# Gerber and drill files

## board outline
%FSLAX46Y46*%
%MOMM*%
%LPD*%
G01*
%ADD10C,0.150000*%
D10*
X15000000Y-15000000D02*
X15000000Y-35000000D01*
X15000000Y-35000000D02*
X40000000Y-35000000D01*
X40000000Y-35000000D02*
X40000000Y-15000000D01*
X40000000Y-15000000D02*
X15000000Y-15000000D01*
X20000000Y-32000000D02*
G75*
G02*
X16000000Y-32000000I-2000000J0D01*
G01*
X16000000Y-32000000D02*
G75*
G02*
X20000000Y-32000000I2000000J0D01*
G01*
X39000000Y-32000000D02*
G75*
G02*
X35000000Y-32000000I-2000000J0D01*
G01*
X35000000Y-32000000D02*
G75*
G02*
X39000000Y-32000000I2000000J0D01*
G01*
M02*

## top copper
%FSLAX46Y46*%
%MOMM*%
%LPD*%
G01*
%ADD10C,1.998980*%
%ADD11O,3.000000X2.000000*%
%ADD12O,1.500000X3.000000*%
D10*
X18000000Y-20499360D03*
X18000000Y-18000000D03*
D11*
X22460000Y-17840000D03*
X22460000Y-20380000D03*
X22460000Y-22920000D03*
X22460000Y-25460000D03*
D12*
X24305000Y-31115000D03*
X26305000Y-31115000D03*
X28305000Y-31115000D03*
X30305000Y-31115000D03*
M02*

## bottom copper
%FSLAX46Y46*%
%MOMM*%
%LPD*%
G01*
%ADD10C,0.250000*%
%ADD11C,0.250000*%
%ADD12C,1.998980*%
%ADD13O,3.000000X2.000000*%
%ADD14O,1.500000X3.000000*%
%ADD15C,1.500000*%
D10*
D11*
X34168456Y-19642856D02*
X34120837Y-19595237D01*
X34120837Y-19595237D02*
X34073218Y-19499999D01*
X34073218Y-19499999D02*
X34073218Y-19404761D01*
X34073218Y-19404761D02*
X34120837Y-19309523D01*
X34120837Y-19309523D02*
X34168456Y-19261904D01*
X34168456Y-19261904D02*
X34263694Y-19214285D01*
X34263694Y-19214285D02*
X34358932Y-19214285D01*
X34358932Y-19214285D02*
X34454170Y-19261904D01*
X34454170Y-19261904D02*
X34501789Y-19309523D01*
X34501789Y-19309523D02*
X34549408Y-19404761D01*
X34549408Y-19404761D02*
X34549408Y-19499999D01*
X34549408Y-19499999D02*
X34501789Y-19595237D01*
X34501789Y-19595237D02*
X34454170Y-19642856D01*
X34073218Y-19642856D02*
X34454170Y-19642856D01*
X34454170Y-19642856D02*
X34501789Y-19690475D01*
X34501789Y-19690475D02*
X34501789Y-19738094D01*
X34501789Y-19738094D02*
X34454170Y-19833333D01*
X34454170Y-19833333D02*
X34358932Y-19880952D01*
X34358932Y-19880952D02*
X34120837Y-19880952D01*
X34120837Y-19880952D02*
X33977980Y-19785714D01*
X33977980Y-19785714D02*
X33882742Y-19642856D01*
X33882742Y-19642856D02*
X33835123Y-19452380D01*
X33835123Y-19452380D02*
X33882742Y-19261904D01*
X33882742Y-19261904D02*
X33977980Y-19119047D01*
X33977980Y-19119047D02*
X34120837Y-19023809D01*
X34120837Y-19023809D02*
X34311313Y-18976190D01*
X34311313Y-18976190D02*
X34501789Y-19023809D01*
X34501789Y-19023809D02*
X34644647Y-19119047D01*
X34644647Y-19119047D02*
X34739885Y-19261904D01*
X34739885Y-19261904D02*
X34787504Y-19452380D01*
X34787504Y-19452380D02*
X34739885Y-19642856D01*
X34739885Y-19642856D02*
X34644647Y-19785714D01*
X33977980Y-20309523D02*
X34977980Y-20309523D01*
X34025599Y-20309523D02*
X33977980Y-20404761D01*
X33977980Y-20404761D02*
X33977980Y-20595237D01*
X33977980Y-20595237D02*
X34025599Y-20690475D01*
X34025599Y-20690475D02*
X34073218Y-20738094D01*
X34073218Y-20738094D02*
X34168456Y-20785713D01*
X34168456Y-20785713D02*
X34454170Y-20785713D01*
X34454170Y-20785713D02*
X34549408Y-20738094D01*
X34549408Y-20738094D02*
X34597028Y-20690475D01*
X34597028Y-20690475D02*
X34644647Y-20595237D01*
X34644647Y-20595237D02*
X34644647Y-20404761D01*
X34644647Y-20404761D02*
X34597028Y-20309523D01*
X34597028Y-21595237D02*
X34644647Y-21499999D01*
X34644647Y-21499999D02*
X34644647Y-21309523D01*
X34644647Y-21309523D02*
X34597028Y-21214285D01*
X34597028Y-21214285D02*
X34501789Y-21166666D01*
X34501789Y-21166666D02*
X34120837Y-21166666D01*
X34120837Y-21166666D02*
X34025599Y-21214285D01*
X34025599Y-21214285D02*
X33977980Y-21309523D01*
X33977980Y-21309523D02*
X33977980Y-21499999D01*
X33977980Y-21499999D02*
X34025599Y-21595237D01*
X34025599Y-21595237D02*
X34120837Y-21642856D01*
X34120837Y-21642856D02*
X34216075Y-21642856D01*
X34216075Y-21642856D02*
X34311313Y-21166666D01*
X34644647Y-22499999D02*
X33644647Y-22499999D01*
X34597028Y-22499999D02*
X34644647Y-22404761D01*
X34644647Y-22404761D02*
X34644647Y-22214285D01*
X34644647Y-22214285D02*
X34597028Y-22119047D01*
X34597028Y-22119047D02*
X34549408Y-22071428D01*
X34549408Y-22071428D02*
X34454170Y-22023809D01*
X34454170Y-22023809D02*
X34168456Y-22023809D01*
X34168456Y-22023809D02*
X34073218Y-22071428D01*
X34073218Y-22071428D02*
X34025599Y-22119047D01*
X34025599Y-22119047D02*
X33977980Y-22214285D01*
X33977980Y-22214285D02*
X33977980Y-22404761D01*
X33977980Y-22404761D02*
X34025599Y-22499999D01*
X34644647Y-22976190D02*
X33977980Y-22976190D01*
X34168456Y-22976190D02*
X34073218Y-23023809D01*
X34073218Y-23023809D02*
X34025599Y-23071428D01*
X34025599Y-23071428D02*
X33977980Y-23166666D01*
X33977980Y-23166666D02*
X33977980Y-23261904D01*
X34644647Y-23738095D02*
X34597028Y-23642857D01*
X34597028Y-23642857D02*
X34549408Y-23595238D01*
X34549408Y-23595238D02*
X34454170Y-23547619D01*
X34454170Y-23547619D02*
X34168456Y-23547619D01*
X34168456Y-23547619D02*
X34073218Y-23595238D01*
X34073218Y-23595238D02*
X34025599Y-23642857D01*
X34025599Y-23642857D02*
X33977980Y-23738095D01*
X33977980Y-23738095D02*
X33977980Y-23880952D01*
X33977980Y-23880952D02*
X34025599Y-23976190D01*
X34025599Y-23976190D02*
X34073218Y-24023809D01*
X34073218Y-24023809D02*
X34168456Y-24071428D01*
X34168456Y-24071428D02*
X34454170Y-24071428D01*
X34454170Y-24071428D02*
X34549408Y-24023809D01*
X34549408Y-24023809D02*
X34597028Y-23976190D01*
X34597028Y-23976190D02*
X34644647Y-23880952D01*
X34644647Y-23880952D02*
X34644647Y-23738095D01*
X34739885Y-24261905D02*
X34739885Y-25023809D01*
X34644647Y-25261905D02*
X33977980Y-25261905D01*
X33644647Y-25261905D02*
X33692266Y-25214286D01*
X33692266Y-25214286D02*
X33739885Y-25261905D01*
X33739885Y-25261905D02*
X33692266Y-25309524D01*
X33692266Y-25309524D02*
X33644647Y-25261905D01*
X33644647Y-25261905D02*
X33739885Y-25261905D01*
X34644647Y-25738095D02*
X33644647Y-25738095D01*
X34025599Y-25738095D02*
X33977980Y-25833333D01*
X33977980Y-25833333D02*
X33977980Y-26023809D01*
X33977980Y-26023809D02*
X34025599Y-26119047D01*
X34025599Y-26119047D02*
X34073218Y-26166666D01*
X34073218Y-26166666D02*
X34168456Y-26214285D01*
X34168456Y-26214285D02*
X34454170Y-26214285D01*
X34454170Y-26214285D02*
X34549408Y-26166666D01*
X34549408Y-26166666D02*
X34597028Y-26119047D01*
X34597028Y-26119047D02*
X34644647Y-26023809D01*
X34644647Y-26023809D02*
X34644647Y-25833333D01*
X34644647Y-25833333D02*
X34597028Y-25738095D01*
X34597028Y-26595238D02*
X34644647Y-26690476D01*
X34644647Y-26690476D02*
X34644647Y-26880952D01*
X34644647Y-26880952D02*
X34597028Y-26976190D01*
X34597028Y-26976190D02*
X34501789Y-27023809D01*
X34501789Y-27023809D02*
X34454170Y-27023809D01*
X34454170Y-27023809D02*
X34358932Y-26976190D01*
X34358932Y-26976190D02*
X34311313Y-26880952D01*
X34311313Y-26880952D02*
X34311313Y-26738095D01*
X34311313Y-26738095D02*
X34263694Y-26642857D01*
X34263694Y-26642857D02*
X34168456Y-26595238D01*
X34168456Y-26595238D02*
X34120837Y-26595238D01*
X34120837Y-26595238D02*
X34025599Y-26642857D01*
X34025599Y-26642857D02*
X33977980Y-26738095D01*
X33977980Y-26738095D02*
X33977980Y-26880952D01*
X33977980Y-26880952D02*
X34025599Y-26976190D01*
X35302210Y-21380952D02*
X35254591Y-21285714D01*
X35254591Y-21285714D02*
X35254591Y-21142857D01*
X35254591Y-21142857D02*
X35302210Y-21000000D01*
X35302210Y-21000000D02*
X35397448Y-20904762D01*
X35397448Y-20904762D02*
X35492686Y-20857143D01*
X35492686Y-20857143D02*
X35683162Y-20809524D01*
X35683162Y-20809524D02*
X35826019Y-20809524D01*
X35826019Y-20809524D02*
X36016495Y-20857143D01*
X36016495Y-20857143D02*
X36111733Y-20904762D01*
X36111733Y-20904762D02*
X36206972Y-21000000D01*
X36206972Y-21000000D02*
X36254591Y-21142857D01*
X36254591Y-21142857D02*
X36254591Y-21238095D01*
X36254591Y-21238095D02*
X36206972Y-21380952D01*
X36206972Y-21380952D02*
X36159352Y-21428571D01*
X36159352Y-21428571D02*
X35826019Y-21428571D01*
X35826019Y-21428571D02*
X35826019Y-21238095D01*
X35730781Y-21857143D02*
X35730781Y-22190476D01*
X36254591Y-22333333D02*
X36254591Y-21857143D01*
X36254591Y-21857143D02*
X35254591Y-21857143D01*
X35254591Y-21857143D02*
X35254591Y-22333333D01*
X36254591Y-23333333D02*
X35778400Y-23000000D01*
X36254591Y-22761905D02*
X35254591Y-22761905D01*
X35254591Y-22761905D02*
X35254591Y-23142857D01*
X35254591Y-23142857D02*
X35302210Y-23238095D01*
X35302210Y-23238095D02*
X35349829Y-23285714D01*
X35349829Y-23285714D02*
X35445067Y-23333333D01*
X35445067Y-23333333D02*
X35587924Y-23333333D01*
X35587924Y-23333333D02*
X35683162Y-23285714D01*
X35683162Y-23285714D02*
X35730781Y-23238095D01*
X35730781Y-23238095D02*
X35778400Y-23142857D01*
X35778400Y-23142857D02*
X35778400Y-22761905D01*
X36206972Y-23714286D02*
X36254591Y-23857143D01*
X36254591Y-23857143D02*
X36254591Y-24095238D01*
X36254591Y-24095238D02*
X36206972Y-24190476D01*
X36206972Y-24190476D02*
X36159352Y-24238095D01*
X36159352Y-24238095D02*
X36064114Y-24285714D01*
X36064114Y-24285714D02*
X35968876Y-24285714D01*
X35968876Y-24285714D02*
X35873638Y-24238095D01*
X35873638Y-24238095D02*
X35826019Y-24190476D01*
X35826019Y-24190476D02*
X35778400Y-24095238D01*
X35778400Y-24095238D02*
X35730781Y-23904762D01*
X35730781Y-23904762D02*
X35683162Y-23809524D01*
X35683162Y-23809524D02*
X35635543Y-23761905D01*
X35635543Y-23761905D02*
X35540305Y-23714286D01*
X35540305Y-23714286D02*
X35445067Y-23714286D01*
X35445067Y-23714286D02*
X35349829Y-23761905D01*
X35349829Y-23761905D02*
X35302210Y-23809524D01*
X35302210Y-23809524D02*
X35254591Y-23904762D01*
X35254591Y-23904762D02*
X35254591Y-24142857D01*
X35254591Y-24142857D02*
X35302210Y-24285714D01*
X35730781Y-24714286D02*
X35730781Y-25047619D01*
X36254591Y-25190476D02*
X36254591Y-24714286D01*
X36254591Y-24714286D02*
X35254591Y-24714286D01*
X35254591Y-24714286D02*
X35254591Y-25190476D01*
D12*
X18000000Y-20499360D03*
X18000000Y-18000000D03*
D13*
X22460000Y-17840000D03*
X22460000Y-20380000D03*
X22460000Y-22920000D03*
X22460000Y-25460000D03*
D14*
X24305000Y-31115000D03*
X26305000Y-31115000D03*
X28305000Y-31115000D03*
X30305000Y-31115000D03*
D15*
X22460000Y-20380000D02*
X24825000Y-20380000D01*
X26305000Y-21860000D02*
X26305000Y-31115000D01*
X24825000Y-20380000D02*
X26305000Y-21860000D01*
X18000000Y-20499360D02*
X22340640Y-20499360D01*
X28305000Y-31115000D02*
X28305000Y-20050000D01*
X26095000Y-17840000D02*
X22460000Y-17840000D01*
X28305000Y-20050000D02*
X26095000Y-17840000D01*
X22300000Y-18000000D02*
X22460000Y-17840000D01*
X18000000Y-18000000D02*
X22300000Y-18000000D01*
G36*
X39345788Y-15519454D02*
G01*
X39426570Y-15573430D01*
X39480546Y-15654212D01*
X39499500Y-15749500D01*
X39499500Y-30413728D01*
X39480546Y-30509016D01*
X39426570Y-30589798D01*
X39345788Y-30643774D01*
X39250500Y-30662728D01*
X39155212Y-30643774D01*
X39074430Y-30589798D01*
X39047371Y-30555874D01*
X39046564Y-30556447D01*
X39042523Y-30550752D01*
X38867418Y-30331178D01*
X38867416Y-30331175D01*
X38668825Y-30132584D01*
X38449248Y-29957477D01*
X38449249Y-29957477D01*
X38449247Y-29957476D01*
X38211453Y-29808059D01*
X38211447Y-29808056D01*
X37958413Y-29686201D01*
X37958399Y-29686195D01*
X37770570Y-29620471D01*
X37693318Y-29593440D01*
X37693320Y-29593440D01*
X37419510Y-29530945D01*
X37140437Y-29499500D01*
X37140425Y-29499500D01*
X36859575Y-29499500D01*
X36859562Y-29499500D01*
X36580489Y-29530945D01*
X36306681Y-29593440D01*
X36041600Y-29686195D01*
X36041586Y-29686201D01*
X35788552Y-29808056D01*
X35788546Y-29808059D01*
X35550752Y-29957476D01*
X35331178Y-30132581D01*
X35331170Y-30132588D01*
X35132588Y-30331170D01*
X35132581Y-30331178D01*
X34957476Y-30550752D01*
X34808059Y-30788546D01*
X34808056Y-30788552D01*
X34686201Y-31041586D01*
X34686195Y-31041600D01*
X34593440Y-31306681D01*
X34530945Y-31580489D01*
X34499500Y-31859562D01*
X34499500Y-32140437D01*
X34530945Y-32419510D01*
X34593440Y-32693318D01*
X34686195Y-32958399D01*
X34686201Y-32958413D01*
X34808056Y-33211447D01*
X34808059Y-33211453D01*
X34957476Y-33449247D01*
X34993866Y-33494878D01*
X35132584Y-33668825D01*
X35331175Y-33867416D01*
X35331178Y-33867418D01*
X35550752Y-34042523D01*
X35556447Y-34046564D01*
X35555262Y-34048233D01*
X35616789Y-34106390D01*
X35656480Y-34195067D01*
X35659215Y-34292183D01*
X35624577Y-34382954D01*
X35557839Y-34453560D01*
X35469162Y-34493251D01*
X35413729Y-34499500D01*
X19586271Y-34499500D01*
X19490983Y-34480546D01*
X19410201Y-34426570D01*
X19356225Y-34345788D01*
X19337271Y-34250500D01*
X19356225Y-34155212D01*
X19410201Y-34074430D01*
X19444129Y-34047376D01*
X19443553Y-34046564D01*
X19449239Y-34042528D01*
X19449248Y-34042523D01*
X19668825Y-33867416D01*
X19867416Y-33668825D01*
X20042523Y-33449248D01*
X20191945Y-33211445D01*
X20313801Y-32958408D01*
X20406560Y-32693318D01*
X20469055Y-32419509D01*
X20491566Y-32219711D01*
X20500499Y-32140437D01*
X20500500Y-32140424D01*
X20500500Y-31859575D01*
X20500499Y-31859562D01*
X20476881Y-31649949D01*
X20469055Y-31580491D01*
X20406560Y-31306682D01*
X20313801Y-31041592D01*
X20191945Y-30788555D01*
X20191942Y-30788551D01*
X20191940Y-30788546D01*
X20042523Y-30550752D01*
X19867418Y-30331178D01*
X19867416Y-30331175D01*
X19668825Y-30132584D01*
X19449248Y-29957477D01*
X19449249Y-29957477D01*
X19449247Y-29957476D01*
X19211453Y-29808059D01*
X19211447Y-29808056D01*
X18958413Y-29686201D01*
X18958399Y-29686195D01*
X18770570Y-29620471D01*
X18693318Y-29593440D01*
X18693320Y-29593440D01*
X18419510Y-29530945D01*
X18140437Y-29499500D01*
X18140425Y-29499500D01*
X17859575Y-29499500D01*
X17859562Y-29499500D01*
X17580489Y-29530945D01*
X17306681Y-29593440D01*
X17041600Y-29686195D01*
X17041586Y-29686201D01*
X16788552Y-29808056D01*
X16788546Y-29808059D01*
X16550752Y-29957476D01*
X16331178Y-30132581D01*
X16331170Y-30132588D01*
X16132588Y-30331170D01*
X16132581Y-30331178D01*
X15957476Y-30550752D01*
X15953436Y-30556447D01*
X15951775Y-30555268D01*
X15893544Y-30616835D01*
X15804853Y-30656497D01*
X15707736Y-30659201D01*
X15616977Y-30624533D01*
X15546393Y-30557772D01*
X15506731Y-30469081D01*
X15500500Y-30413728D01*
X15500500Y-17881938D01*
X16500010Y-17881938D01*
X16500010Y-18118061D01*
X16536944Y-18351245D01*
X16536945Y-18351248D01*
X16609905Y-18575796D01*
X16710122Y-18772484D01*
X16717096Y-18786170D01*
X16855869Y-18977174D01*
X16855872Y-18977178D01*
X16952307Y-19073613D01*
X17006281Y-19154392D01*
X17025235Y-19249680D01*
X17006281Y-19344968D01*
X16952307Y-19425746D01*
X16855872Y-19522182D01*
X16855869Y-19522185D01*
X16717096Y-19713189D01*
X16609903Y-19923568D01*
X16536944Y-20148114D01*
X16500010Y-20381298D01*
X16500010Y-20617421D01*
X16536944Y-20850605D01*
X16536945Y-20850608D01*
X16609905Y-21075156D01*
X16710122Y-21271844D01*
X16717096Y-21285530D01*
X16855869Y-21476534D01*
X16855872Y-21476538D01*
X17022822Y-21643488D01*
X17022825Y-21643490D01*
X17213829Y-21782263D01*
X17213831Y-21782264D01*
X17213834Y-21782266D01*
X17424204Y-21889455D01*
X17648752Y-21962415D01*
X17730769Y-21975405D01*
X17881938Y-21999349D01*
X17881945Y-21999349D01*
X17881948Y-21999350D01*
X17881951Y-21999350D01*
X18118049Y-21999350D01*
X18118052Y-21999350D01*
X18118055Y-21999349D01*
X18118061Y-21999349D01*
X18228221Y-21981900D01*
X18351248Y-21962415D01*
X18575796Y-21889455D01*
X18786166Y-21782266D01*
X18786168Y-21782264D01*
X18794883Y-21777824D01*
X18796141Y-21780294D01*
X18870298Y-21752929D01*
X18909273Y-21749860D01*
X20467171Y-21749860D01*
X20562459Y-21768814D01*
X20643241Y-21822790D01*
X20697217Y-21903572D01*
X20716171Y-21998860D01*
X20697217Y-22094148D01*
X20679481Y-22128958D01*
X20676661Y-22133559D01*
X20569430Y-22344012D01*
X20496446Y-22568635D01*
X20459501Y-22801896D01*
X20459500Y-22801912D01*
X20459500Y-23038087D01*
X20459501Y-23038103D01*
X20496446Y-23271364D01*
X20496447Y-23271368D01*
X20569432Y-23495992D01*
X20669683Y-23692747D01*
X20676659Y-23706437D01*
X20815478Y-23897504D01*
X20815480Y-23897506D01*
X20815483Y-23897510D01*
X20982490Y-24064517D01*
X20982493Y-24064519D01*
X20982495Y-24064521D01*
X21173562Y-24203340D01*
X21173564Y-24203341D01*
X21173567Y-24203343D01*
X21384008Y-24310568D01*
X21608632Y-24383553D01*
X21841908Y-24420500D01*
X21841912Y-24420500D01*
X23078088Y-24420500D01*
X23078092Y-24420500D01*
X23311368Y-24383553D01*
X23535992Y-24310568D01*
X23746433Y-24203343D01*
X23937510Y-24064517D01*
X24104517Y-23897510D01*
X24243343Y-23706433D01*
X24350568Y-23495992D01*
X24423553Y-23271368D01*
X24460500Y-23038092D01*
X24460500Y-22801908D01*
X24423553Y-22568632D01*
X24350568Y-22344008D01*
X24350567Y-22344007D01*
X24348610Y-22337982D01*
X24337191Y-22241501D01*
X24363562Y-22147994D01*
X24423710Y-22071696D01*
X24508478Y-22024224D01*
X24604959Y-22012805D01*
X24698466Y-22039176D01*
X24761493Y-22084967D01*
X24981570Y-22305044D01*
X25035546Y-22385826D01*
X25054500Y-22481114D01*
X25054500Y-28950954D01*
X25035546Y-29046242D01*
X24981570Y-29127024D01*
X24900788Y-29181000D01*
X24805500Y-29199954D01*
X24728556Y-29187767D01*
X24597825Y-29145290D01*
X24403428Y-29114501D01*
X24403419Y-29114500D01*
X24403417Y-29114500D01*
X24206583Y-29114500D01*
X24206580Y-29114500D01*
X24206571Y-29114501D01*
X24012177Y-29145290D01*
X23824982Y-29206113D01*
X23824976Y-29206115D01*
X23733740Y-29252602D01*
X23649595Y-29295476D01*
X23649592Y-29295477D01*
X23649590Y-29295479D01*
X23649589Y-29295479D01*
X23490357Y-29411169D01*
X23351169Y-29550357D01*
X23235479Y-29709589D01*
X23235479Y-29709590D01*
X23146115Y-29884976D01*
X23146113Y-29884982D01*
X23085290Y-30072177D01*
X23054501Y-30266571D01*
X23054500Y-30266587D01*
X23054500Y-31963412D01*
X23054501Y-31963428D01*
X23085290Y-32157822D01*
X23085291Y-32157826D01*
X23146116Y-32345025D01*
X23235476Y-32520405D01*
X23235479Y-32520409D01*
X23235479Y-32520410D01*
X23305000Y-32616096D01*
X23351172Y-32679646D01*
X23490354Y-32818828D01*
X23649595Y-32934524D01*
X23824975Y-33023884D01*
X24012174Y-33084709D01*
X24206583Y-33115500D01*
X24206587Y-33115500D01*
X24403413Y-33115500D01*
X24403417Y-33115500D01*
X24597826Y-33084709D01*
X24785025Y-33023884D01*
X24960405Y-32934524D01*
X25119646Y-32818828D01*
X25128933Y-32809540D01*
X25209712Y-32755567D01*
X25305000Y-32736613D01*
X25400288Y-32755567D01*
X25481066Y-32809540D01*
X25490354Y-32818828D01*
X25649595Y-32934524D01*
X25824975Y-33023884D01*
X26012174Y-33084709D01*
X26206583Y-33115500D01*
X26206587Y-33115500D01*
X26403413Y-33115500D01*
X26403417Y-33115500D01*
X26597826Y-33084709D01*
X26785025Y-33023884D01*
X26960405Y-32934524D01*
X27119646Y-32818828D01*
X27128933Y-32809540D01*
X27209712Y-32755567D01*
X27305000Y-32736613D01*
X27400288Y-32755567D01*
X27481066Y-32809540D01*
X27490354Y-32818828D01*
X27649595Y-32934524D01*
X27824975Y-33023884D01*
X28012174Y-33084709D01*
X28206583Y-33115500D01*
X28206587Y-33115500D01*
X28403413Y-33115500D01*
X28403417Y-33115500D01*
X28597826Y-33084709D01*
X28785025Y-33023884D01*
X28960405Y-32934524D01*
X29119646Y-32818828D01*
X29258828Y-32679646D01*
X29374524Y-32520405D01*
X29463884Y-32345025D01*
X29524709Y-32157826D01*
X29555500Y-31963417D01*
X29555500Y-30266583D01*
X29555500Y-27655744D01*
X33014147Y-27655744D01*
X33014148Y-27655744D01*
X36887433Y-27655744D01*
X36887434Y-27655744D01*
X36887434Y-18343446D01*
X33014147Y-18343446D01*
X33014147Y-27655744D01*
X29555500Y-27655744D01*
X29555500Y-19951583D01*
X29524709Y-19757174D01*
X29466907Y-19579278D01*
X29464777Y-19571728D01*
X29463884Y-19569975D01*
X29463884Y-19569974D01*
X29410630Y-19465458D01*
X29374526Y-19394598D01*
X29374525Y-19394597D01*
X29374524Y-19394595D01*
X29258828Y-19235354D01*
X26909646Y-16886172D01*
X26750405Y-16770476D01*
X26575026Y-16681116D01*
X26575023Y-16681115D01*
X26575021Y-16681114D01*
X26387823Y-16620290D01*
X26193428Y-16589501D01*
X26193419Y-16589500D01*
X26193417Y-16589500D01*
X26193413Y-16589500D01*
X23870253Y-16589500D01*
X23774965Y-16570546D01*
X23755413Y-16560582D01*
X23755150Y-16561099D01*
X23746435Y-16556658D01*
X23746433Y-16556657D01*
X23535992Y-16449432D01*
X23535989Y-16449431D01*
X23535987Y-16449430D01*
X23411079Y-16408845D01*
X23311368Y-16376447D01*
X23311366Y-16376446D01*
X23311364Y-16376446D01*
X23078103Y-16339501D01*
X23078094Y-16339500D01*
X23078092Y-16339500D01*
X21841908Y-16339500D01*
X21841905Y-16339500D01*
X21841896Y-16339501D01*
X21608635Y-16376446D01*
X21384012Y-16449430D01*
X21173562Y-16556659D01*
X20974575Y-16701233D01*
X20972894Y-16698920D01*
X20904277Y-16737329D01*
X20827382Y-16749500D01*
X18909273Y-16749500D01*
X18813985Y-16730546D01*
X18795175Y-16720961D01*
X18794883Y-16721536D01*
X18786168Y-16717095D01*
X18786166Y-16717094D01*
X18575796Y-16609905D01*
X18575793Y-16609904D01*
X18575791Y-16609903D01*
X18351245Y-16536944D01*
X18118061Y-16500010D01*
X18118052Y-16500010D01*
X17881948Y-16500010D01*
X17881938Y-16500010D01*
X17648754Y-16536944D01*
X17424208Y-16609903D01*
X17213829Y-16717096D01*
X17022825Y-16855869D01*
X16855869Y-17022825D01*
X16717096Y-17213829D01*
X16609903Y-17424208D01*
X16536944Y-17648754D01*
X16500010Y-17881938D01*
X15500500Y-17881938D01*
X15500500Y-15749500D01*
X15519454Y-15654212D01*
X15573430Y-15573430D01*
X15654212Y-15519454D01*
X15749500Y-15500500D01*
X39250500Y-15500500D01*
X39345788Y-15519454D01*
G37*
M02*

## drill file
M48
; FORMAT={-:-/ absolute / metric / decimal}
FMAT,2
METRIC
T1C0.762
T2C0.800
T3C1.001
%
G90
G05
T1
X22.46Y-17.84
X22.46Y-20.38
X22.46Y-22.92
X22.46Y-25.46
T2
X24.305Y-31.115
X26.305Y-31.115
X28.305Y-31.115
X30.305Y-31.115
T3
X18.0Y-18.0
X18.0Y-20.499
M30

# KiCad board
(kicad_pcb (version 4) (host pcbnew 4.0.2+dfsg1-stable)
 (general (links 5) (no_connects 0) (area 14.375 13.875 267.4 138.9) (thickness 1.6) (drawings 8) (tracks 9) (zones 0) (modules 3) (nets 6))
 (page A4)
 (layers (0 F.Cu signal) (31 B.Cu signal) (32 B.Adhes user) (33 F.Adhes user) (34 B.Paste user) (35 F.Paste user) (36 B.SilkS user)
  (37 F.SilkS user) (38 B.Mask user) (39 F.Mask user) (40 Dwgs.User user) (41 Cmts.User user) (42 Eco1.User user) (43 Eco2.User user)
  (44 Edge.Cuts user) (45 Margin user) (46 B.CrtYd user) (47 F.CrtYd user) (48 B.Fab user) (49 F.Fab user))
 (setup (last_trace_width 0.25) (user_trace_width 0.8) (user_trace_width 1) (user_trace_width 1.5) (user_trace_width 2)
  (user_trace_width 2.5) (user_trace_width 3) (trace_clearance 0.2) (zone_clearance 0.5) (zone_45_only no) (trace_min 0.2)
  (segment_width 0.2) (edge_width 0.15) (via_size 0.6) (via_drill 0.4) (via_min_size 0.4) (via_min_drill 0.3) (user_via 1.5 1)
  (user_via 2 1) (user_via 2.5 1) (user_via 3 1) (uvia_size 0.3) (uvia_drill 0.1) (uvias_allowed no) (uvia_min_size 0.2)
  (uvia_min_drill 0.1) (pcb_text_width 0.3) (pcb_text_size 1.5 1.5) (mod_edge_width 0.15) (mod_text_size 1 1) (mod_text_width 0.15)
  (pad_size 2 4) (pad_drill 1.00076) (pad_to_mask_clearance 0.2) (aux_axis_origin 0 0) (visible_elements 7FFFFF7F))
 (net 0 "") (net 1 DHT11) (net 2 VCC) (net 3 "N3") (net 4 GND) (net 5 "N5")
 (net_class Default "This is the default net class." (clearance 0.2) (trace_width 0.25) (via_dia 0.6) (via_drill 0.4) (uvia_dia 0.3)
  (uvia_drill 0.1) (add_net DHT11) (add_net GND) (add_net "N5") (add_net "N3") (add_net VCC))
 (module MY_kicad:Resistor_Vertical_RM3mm (layer F.Cu) (at 18 18 90)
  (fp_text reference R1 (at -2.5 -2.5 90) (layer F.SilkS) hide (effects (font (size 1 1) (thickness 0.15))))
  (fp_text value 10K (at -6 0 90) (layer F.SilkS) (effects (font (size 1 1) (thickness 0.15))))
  (pad 1 thru_hole circle (at -2.49936 0 90) (size 1.99898 1.99898) (drill 1.00076) (layers *.Cu *.SilkS *.Mask) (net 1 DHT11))
  (pad 2 thru_hole circle (at 0 0 90) (size 1.99898 1.99898) (drill 1.00076) (layers *.Cu *.SilkS *.Mask) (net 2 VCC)))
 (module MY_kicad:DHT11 (layer F.Cu) (at 25 28)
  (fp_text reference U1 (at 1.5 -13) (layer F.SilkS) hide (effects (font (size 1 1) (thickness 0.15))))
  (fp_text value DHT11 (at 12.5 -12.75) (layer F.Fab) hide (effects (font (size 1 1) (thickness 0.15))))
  (pad 1 thru_hole oval (at -2.54 -10.16) (size 3 2) (drill 0.762) (layers *.Cu B.Mask) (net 2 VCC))
  (pad 2 thru_hole oval (at -2.54 -7.62) (size 3 2) (drill 0.762) (layers *.Cu B.Mask) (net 1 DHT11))
  (pad 3 thru_hole oval (at -2.54 -5.08) (size 3 2) (drill 0.762) (layers *.Cu B.Mask) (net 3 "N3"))
  (pad 4 thru_hole oval (at -2.54 -2.54) (size 3 2) (drill 0.762) (layers *.Cu B.Mask) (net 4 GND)))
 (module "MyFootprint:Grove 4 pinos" (layer F.Cu) (at 27.305 31.115)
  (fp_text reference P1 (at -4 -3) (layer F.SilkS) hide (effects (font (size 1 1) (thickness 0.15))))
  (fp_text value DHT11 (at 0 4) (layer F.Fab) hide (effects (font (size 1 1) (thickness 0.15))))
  (pad 1 thru_hole oval (at -3 0) (size 1.5 3) (drill 0.8) (layers *.Cu) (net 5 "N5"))
  (pad 2 thru_hole oval (at -1 0) (size 1.5 3) (drill 0.8) (layers *.Cu) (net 1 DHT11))
  (pad 3 thru_hole oval (at 1 0) (size 1.5 3) (drill 0.8) (layers *.Cu) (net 2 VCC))
  (pad 4 thru_hole oval (at 3 0) (size 1.5 3) (drill 0.8) (layers *.Cu) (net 4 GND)))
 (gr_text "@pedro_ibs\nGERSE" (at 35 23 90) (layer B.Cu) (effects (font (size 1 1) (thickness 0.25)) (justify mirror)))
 (gr_line (start 15 15) (end 15 35) (angle 90) (layer Edge.Cuts) (width 0.15))
 (gr_line (start 15 35) (end 40 35) (angle 90) (layer Edge.Cuts) (width 0.15))
 (gr_line (start 40 35) (end 40 15) (angle 90) (layer Edge.Cuts) (width 0.15))
 (gr_line (start 40 15) (end 15 15) (angle 90) (layer Edge.Cuts) (width 0.15))
 (gr_circle (center 18 32) (end 20 32) (layer Edge.Cuts) (width 0.15))
 (gr_circle (center 37 32) (end 39 32) (layer Edge.Cuts) (width 0.15))
 (segment (start 22.46 20.38) (end 24.825 20.38) (width 1.5) (layer B.Cu) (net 1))
 (segment (start 26.305 21.86) (end 26.305 31.115) (width 1.5) (layer B.Cu) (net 1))
 (segment (start 24.825 20.38) (end 26.305 21.86) (width 1.5) (layer B.Cu) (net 1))
 (segment (start 18 20.49936) (end 22.34064 20.49936) (width 1.5) (layer B.Cu) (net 1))
 (segment (start 28.305 31.115) (end 28.305 20.05) (width 1.5) (layer B.Cu) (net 2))
 (segment (start 26.095 17.84) (end 22.46 17.84) (width 1.5) (layer B.Cu) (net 2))
 (segment (start 28.305 20.05) (end 26.095 17.84) (width 1.5) (layer B.Cu) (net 2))
 (segment (start 22.3 18) (end 22.46 17.84) (width 1.5) (layer B.Cu) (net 2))
 (segment (start 18 18) (end 22.3 18) (width 1.5) (layer B.Cu) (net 2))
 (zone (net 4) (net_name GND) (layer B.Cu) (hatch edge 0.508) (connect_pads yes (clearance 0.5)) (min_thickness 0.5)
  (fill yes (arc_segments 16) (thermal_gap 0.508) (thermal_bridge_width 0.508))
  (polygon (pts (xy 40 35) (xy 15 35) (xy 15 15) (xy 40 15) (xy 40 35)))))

